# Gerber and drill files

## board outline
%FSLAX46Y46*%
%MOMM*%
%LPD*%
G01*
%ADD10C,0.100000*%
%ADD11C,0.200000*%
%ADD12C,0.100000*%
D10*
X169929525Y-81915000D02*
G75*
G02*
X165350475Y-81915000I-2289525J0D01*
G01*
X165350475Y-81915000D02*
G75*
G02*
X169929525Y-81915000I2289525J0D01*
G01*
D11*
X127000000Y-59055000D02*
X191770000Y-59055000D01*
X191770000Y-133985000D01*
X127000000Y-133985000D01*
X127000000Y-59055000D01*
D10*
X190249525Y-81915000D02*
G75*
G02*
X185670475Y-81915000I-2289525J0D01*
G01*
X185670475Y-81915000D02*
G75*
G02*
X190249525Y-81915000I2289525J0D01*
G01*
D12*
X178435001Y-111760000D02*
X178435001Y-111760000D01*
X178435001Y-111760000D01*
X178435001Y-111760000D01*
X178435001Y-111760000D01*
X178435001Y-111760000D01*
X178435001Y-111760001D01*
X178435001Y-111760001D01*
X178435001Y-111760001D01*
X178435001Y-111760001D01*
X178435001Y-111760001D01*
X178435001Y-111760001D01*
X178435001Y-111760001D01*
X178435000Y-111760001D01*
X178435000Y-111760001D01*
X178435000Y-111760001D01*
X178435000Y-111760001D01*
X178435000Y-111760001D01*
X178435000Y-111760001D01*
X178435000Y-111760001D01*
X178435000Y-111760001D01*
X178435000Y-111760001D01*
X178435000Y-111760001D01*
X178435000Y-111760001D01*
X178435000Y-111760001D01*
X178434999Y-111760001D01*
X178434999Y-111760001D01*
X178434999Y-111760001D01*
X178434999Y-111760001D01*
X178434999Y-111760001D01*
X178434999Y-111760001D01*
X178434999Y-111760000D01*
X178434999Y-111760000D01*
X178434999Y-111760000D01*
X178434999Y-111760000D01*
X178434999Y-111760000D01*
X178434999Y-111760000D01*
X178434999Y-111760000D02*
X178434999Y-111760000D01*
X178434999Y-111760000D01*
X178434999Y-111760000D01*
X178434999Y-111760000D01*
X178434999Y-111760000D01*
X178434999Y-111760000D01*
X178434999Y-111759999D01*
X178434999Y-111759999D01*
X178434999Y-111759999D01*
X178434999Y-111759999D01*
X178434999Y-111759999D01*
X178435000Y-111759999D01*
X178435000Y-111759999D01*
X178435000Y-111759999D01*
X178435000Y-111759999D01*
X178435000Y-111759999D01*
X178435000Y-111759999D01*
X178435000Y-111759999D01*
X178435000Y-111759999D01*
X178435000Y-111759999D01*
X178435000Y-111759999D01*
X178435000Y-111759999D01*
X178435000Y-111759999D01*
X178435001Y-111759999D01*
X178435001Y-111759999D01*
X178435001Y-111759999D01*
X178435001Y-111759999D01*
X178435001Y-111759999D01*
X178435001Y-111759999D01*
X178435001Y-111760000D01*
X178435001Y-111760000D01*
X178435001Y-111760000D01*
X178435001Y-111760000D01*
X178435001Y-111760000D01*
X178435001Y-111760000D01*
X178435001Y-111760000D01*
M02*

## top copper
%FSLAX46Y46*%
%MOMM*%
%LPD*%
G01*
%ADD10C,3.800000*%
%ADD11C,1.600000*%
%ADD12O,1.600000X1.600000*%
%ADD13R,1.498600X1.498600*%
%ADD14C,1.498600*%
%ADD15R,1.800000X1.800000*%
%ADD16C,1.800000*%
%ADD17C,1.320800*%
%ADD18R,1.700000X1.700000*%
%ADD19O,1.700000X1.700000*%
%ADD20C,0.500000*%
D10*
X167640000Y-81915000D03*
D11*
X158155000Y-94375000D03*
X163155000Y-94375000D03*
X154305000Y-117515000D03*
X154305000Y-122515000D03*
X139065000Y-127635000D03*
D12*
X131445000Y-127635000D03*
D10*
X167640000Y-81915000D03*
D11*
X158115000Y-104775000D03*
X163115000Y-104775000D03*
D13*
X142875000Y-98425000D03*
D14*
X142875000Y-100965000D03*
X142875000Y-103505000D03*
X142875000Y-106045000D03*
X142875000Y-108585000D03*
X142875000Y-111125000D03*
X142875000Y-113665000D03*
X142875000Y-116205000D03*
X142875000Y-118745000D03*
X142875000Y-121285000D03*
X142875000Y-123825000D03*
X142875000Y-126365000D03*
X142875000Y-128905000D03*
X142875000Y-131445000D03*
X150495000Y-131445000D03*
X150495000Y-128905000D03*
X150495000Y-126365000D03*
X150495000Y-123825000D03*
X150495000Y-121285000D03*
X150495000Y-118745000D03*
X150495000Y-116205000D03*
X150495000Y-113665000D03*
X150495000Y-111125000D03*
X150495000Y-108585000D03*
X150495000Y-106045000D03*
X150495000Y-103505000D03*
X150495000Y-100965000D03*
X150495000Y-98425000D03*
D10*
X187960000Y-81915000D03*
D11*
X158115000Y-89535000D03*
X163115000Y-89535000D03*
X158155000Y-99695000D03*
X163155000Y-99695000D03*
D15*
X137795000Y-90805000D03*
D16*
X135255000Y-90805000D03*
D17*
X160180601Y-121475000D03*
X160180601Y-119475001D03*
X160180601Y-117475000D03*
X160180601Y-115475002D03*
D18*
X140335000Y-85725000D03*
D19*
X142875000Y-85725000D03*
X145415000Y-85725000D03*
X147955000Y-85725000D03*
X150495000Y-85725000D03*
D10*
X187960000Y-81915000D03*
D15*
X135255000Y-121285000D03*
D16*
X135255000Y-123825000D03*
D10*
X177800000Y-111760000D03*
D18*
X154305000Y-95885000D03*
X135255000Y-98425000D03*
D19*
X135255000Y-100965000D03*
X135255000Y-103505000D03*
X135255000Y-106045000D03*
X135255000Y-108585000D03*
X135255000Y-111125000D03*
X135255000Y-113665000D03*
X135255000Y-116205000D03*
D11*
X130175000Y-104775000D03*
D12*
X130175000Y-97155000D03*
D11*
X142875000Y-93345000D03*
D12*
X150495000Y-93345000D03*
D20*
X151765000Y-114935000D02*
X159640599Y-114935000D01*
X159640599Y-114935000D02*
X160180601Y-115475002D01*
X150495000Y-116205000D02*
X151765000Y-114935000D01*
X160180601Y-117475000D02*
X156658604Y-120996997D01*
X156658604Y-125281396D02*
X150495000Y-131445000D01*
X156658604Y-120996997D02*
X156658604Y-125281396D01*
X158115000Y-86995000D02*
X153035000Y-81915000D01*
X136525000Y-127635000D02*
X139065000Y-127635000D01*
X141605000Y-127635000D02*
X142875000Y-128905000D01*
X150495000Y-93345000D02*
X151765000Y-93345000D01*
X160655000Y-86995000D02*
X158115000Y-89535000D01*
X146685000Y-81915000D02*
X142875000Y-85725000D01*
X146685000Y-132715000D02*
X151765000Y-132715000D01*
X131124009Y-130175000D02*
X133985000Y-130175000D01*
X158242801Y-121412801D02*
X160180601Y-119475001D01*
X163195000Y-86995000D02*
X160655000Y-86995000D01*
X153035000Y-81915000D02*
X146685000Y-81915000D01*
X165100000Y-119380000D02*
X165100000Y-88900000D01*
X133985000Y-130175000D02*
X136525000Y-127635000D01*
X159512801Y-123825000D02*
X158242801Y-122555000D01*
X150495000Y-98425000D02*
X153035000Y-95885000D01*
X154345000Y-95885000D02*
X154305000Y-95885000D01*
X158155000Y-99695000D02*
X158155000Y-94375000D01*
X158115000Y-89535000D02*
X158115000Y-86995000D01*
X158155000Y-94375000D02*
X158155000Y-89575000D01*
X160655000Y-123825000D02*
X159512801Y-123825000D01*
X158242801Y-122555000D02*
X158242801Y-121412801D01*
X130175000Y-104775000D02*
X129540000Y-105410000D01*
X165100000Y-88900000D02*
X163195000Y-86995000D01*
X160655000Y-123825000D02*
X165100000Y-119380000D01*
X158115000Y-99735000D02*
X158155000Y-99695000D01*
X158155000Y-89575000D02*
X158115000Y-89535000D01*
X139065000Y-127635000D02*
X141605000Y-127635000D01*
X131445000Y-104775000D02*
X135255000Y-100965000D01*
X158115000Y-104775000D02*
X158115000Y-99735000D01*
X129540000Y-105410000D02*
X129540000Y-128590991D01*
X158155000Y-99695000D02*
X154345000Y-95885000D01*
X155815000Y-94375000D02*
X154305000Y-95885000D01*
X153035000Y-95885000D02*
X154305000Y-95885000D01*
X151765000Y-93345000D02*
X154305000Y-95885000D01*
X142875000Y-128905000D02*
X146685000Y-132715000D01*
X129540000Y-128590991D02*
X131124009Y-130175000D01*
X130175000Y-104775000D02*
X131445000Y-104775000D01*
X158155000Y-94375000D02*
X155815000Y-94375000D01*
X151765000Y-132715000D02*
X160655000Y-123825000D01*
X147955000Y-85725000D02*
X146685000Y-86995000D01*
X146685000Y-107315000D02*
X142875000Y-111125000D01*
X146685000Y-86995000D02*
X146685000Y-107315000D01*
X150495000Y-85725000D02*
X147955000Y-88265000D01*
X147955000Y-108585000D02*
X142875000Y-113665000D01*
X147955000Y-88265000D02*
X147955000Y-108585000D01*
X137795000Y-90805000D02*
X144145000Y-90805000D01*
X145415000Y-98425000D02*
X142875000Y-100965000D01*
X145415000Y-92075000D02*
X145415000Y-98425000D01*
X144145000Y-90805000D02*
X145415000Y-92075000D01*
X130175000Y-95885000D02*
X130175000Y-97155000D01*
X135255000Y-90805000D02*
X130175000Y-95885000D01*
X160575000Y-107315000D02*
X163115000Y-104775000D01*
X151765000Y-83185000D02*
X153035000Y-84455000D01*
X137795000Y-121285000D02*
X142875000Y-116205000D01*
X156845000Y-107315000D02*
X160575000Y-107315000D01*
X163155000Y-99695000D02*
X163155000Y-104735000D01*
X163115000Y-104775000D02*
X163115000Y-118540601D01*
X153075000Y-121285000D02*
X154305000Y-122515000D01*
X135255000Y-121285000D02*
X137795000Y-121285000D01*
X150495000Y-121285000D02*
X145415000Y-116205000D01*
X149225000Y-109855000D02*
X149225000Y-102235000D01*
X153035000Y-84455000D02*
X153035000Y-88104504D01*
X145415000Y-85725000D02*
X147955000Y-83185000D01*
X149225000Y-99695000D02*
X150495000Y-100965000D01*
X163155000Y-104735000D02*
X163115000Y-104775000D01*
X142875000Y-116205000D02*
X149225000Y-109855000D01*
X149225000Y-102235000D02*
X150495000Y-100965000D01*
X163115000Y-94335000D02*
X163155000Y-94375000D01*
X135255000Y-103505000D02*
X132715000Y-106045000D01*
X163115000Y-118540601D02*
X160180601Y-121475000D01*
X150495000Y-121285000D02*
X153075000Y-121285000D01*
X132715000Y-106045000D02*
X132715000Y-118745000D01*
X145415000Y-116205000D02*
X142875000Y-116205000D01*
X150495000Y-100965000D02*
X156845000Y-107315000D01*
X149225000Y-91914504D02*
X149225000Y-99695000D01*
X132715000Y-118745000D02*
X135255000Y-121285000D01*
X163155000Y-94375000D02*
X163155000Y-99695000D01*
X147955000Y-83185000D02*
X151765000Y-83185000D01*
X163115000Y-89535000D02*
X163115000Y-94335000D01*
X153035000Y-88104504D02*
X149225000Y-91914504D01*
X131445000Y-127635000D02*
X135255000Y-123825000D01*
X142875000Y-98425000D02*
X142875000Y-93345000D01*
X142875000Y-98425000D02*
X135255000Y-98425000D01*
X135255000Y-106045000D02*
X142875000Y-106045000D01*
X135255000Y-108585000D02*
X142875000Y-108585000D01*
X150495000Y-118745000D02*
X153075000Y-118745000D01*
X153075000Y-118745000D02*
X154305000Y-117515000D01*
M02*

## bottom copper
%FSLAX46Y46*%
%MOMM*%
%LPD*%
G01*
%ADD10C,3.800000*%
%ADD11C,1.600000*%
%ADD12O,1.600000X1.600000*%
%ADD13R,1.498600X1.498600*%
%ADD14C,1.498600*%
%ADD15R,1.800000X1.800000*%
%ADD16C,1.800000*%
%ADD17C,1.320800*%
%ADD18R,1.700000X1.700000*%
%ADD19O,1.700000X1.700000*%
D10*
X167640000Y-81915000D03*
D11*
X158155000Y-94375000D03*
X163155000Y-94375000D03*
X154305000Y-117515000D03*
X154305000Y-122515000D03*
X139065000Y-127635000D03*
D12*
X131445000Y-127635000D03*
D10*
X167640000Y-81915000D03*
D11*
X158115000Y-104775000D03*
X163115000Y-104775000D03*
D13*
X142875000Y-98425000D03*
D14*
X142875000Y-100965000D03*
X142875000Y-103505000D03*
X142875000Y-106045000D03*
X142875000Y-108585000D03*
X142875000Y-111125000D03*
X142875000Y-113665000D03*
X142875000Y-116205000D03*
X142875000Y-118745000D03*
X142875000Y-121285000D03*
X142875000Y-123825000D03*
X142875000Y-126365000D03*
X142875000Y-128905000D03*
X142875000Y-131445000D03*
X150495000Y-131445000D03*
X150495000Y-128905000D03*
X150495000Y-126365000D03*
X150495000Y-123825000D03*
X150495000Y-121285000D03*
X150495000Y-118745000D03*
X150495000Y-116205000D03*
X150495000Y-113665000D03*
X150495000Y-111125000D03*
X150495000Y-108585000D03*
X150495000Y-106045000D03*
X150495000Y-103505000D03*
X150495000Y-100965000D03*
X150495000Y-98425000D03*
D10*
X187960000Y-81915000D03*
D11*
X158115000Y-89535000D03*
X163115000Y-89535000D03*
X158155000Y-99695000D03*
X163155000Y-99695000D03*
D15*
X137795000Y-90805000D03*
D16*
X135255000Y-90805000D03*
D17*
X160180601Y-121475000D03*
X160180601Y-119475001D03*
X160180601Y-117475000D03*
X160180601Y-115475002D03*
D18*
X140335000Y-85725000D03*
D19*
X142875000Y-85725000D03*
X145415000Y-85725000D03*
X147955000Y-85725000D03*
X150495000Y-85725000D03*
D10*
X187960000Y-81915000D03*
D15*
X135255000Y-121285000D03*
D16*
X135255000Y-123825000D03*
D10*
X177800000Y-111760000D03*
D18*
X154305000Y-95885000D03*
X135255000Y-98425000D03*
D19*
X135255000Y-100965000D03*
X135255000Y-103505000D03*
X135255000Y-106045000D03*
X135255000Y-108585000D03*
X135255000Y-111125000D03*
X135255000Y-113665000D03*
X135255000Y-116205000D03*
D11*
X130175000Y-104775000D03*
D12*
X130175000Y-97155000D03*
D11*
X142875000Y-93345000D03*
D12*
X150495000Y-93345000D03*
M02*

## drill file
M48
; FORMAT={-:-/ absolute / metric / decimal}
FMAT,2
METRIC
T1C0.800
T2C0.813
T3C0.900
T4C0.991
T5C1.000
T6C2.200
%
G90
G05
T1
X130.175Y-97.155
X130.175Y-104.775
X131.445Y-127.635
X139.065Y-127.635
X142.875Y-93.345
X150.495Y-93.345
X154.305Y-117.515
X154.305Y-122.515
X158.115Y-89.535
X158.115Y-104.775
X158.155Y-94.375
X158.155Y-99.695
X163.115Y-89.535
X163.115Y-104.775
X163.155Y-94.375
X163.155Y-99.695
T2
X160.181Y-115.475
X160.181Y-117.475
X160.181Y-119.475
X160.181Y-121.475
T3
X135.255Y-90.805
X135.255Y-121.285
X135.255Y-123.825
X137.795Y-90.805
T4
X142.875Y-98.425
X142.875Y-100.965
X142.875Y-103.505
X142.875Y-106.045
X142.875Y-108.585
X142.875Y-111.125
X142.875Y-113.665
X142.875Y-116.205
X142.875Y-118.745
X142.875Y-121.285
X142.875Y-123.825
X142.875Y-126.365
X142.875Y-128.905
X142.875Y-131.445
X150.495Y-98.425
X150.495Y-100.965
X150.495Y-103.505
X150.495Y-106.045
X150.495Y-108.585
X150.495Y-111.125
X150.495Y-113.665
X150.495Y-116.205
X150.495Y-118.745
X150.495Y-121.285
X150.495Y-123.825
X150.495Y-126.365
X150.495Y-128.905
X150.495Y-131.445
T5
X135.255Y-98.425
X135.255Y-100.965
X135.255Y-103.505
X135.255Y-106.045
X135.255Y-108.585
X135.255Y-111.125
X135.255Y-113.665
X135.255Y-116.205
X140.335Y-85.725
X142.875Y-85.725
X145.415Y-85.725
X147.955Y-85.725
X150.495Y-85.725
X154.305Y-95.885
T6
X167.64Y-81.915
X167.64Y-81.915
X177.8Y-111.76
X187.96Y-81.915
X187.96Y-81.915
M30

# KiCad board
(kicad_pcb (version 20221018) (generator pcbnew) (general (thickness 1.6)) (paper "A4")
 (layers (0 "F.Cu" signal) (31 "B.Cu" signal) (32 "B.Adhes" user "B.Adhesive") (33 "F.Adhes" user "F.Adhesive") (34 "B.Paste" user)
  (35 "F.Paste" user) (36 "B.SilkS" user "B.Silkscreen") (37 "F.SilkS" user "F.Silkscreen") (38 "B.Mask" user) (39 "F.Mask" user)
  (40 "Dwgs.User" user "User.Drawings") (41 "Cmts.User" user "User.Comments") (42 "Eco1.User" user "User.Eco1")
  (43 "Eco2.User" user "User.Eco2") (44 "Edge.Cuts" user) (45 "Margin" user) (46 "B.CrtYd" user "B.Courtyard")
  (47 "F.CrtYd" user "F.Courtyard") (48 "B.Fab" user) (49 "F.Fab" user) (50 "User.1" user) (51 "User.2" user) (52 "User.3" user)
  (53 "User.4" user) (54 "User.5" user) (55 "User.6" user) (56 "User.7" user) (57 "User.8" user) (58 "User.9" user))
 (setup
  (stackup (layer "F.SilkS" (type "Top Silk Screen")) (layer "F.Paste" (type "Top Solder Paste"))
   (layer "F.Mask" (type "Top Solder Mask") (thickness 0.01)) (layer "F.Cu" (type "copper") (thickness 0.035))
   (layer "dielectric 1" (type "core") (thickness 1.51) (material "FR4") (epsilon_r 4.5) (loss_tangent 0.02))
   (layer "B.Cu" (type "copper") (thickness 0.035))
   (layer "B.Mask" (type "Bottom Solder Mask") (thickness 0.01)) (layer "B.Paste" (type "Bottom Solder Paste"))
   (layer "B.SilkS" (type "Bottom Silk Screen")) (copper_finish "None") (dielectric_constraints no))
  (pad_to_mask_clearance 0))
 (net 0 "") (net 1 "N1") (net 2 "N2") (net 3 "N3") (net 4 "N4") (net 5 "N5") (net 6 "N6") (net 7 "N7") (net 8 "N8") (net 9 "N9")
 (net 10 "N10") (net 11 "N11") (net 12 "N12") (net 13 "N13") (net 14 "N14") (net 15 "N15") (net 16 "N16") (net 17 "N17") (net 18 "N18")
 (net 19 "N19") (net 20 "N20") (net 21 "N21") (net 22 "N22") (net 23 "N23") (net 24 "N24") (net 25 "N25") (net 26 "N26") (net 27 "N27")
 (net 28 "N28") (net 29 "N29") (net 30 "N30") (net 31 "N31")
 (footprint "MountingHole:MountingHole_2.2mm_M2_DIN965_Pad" (layer "F.Cu") (at 167.64 81.915)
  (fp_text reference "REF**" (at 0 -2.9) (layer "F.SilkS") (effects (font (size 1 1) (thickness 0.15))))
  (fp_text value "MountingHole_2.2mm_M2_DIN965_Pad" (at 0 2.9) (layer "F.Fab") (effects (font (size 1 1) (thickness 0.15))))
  (pad "1" thru_hole circle (at 0 0) (size 3.8 3.8) (drill 2.2) (layers "*.Cu" "*.Mask")))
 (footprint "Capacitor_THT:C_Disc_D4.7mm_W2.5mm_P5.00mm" (layer "F.Cu") (at 158.155 94.375)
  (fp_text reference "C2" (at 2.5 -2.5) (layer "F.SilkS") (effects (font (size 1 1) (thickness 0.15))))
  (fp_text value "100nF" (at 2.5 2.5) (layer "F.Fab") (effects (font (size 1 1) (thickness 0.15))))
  (pad "1" thru_hole circle (at 0 0) (size 1.6 1.6) (drill 0.8) (layers "*.Cu" "*.Mask") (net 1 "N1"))
  (pad "2" thru_hole circle (at 5 0) (size 1.6 1.6) (drill 0.8) (layers "*.Cu" "*.Mask") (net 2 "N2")))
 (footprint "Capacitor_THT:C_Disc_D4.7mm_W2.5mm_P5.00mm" (layer "F.Cu") (at 154.305 117.515 -90)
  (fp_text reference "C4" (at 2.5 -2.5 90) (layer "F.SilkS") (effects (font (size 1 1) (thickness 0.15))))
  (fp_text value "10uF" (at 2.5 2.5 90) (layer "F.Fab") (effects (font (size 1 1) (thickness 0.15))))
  (pad "1" thru_hole circle (at 0 0 270) (size 1.6 1.6) (drill 0.8) (layers "*.Cu" "*.Mask") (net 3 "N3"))
  (pad "2" thru_hole circle (at 5 0 270) (size 1.6 1.6) (drill 0.8) (layers "*.Cu" "*.Mask") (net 2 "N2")))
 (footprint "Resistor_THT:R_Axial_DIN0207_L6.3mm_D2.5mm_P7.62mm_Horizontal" (layer "F.Cu") (at 139.065 127.635 180)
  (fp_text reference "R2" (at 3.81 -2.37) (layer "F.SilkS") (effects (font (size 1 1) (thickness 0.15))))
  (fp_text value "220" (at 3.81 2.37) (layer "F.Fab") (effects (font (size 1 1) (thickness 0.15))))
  (pad "1" thru_hole circle (at 0 0 180) (size 1.6 1.6) (drill 0.8) (layers "*.Cu" "*.Mask") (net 1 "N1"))
  (pad "2" thru_hole oval (at 7.62 0 180) (size 1.6 1.6) (drill 0.8) (layers "*.Cu" "*.Mask") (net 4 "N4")))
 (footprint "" (layer "F.Cu") (at 167.64 81.915)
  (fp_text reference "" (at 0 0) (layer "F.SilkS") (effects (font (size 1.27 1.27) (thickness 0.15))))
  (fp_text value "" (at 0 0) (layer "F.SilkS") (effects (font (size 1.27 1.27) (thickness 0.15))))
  (pad "1" thru_hole circle (at 0 0) (size 3.8 3.8) (drill 2.2) (layers "*.Cu" "*.Mask")))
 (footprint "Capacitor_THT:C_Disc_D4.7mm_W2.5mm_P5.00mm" (layer "F.Cu") (at 158.115 104.775)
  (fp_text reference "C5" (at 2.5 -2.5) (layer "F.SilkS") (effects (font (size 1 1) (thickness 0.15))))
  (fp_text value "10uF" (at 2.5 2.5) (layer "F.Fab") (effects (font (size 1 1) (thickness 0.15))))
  (pad "1" thru_hole circle (at 0 0) (size 1.6 1.6) (drill 0.8) (layers "*.Cu" "*.Mask") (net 1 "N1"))
  (pad "2" thru_hole circle (at 5 0) (size 1.6 1.6) (drill 0.8) (layers "*.Cu" "*.Mask") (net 2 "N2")))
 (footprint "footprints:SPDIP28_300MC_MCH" (layer "F.Cu") (at 142.875 98.425)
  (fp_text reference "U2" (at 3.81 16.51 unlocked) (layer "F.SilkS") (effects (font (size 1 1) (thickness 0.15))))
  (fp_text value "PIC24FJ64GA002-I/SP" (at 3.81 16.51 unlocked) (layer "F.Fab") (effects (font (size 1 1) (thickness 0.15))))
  (pad "1" thru_hole rect (at 0 0) (size 1.4986 1.4986) (drill 0.9906) (layers "*.Cu" "*.Mask") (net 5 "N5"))
  (pad "2" thru_hole circle (at 0 2.54) (size 1.4986 1.4986) (drill 0.9906) (layers "*.Cu" "*.Mask") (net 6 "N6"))
  (pad "3" thru_hole circle (at 0 5.08) (size 1.4986 1.4986) (drill 0.9906) (layers "*.Cu" "*.Mask") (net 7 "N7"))
  (pad "4" thru_hole circle (at 0 7.62) (size 1.4986 1.4986) (drill 0.9906) (layers "*.Cu" "*.Mask") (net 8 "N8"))
  (pad "5" thru_hole circle (at 0 10.16) (size 1.4986 1.4986) (drill 0.9906) (layers "*.Cu" "*.Mask") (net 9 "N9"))
  (pad "6" thru_hole circle (at 0 12.7) (size 1.4986 1.4986) (drill 0.9906) (layers "*.Cu" "*.Mask") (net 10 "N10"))
  (pad "7" thru_hole circle (at 0 15.24) (size 1.4986 1.4986) (drill 0.9906) (layers "*.Cu" "*.Mask") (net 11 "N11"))
  (pad "8" thru_hole circle (at 0 17.78) (size 1.4986 1.4986) (drill 0.9906) (layers "*.Cu" "*.Mask") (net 2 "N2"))
  (pad "9" thru_hole circle (at 0 20.32) (size 1.4986 1.4986) (drill 0.9906) (layers "*.Cu" "*.Mask") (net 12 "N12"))
  (pad "10" thru_hole circle (at 0 22.86) (size 1.4986 1.4986) (drill 0.9906) (layers "*.Cu" "*.Mask") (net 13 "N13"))
  (pad "11" thru_hole circle (at 0 25.4) (size 1.4986 1.4986) (drill 0.9906) (layers "*.Cu" "*.Mask") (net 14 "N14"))
  (pad "12" thru_hole circle (at 0 27.94) (size 1.4986 1.4986) (drill 0.9906) (layers "*.Cu" "*.Mask") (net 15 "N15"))
  (pad "13" thru_hole circle (at 0 30.48) (size 1.4986 1.4986) (drill 0.9906) (layers "*.Cu" "*.Mask") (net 1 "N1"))
  (pad "14" thru_hole circle (at 0 33.02) (size 1.4986 1.4986) (drill 0.9906) (layers "*.Cu" "*.Mask") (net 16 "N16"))
  (pad "15" thru_hole circle (at 7.62 33.02) (size 1.4986 1.4986) (drill 0.9906) (layers "*.Cu" "*.Mask") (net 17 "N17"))
  (pad "16" thru_hole circle (at 7.62 30.48) (size 1.4986 1.4986) (drill 0.9906) (layers "*.Cu" "*.Mask") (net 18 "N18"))
  (pad "17" thru_hole circle (at 7.62 27.94) (size 1.4986 1.4986) (drill 0.9906) (layers "*.Cu" "*.Mask") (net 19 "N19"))
  (pad "18" thru_hole circle (at 7.62 25.4) (size 1.4986 1.4986) (drill 0.9906) (layers "*.Cu" "*.Mask") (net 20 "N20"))
  (pad "19" thru_hole circle (at 7.62 22.86) (size 1.4986 1.4986) (drill 0.9906) (layers "*.Cu" "*.Mask") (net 2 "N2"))
  (pad "20" thru_hole circle (at 7.62 20.32) (size 1.4986 1.4986) (drill 0.9906) (layers "*.Cu" "*.Mask") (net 3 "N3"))
  (pad "21" thru_hole circle (at 7.62 17.78) (size 1.4986 1.4986) (drill 0.9906) (layers "*.Cu" "*.Mask") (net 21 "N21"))
  (pad "22" thru_hole circle (at 7.62 15.24) (size 1.4986 1.4986) (drill 0.9906) (layers "*.Cu" "*.Mask") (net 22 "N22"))
  (pad "23" thru_hole circle (at 7.62 12.7) (size 1.4986 1.4986) (drill 0.9906) (layers "*.Cu" "*.Mask") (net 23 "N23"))
  (pad "24" thru_hole circle (at 7.62 10.16) (size 1.4986 1.4986) (drill 0.9906) (layers "*.Cu" "*.Mask") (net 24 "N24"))
  (pad "25" thru_hole circle (at 7.62 7.62) (size 1.4986 1.4986) (drill 0.9906) (layers "*.Cu" "*.Mask") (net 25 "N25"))
  (pad "26" thru_hole circle (at 7.62 5.08) (size 1.4986 1.4986) (drill 0.9906) (layers "*.Cu" "*.Mask") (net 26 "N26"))
  (pad "27" thru_hole circle (at 7.62 2.54) (size 1.4986 1.4986) (drill 0.9906) (layers "*.Cu" "*.Mask") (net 2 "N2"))
  (pad "28" thru_hole circle (at 7.62 0) (size 1.4986 1.4986) (drill 0.9906) (layers "*.Cu" "*.Mask") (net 1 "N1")))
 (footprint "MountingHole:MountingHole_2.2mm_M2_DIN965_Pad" (layer "F.Cu") (at 187.96 81.915)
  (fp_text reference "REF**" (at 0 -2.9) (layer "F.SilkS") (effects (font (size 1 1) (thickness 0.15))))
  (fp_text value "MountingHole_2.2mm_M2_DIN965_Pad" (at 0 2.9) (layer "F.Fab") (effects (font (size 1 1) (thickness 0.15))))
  (pad "1" thru_hole circle (at 0 0) (size 3.8 3.8) (drill 2.2) (layers "*.Cu" "*.Mask")))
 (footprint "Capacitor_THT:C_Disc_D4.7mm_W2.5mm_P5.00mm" (layer "F.Cu") (at 158.115 89.535)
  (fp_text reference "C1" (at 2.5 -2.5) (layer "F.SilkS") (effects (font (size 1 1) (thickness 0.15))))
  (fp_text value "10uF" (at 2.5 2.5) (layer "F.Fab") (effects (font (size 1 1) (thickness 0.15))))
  (pad "1" thru_hole circle (at 0 0) (size 1.6 1.6) (drill 0.8) (layers "*.Cu" "*.Mask") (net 1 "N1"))
  (pad "2" thru_hole circle (at 5 0) (size 1.6 1.6) (drill 0.8) (layers "*.Cu" "*.Mask") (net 2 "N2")))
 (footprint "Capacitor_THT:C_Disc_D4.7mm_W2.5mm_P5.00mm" (layer "F.Cu") (at 158.155 99.695)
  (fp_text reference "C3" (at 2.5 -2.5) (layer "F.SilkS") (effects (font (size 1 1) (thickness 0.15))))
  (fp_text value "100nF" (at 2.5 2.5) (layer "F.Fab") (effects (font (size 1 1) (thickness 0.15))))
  (pad "1" thru_hole circle (at 0 0) (size 1.6 1.6) (drill 0.8) (layers "*.Cu" "*.Mask") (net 1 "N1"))
  (pad "2" thru_hole circle (at 5 0) (size 1.6 1.6) (drill 0.8) (layers "*.Cu" "*.Mask") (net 2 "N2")))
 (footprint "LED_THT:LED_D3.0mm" (layer "F.Cu") (at 137.795 90.805 180)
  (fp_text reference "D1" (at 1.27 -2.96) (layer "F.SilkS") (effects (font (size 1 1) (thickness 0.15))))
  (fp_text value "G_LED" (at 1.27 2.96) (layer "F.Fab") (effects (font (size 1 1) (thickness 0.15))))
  (pad "1" thru_hole rect (at 0 0 180) (size 1.8 1.8) (drill 0.9) (layers "*.Cu" "*.Mask") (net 6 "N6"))
  (pad "2" thru_hole circle (at 2.54 0 180) (size 1.8 1.8) (drill 0.9) (layers "*.Cu" "*.Mask") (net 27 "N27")))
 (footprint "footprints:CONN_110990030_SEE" (layer "F.Cu") (at 160.180601 121.475 90)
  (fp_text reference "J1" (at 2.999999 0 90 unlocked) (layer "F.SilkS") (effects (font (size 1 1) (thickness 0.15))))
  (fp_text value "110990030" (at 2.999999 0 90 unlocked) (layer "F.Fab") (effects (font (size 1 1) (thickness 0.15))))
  (pad "1" thru_hole circle (at 0 0 90) (size 1.3208 1.3208) (drill 0.8128) (layers "*.Cu" "*.Mask") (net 2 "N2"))
  (pad "2" thru_hole circle (at 1.999999 0 90) (size 1.3208 1.3208) (drill 0.8128) (layers "*.Cu" "*.Mask") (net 1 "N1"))
  (pad "3" thru_hole circle (at 4 0 90) (size 1.3208 1.3208) (drill 0.8128) (layers "*.Cu" "*.Mask") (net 17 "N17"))
  (pad "4" thru_hole circle (at 5.999998 0 90) (size 1.3208 1.3208) (drill 0.8128) (layers "*.Cu" "*.Mask") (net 21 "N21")))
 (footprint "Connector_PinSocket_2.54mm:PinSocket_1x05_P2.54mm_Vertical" (layer "F.Cu") (at 140.335 85.725 90)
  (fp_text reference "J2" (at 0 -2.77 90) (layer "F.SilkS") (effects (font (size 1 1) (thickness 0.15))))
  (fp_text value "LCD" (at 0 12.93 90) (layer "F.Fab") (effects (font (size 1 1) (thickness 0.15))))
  (pad "1" thru_hole rect (at 0 0 90) (size 1.7 1.7) (drill 1) (layers "*.Cu" "*.Mask") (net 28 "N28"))
  (pad "2" thru_hole oval (at 0 2.54 90) (size 1.7 1.7) (drill 1) (layers "*.Cu" "*.Mask") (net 1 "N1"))
  (pad "3" thru_hole oval (at 0 5.08 90) (size 1.7 1.7) (drill 1) (layers "*.Cu" "*.Mask") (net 2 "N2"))
  (pad "4" thru_hole oval (at 0 7.62 90) (size 1.7 1.7) (drill 1) (layers "*.Cu" "*.Mask") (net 10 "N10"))
  (pad "5" thru_hole oval (at 0 10.16 90) (size 1.7 1.7) (drill 1) (layers "*.Cu" "*.Mask") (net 11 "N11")))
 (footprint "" (layer "F.Cu") (at 187.96 81.915)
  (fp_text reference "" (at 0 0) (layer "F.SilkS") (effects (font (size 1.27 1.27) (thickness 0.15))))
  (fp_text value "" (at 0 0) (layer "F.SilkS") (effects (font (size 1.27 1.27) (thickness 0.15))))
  (pad "1" thru_hole circle (at 0 0) (size 3.8 3.8) (drill 2.2) (layers "*.Cu" "*.Mask")))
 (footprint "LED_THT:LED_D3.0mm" (layer "F.Cu") (at 135.255 121.285 -90)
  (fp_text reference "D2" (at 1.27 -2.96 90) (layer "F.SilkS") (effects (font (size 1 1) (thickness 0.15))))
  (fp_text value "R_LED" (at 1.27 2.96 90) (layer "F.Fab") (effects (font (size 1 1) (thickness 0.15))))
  (pad "1" thru_hole rect (at 0 0 270) (size 1.8 1.8) (drill 0.9) (layers "*.Cu" "*.Mask") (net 2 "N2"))
  (pad "2" thru_hole circle (at 2.54 0 270) (size 1.8 1.8) (drill 0.9) (layers "*.Cu" "*.Mask") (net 4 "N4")))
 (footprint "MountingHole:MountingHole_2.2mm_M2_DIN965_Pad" (layer "F.Cu") (at 177.8 111.76)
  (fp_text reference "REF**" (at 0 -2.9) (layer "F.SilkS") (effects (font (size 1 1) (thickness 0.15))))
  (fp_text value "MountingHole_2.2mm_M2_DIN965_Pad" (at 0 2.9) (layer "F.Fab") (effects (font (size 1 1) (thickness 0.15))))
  (pad "1" thru_hole circle (at 0 0) (size 3.8 3.8) (drill 2.2) (layers "*.Cu" "*.Mask")))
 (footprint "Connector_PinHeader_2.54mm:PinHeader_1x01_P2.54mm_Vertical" (layer "F.Cu") (at 154.305 95.885)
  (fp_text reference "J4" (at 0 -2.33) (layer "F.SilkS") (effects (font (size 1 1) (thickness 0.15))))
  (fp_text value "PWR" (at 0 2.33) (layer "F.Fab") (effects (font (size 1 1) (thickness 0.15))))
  (pad "1" thru_hole rect (at 0 0) (size 1.7 1.7) (drill 1) (layers "*.Cu" "*.Mask") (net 1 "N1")))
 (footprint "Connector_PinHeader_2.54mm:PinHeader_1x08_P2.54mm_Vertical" (layer "F.Cu") (at 135.255 98.425)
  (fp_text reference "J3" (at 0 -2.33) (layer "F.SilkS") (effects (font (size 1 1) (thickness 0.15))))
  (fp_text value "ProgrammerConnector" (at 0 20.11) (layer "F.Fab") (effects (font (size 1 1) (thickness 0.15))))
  (pad "1" thru_hole rect (at 0 0) (size 1.7 1.7) (drill 1) (layers "*.Cu" "*.Mask") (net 5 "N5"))
  (pad "2" thru_hole oval (at 0 2.54) (size 1.7 1.7) (drill 1) (layers "*.Cu" "*.Mask") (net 1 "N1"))
  (pad "3" thru_hole oval (at 0 5.08) (size 1.7 1.7) (drill 1) (layers "*.Cu" "*.Mask") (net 2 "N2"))
  (pad "4" thru_hole oval (at 0 7.62) (size 1.7 1.7) (drill 1) (layers "*.Cu" "*.Mask") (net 8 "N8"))
  (pad "5" thru_hole oval (at 0 10.16) (size 1.7 1.7) (drill 1) (layers "*.Cu" "*.Mask") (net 9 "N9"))
  (pad "6" thru_hole oval (at 0 12.7) (size 1.7 1.7) (drill 1) (layers "*.Cu" "*.Mask") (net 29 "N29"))
  (pad "7" thru_hole oval (at 0 15.24) (size 1.7 1.7) (drill 1) (layers "*.Cu" "*.Mask") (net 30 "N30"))
  (pad "8" thru_hole oval (at 0 17.78) (size 1.7 1.7) (drill 1) (layers "*.Cu" "*.Mask") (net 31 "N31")))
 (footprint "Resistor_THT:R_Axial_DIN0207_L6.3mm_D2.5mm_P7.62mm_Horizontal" (layer "F.Cu") (at 130.175 104.775 90)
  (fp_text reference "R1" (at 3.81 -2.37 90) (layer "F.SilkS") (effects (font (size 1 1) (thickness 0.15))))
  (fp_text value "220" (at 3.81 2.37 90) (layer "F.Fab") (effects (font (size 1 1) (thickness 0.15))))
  (pad "1" thru_hole circle (at 0 0 90) (size 1.6 1.6) (drill 0.8) (layers "*.Cu" "*.Mask") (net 1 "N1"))
  (pad "2" thru_hole oval (at 7.62 0 90) (size 1.6 1.6) (drill 0.8) (layers "*.Cu" "*.Mask") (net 27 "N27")))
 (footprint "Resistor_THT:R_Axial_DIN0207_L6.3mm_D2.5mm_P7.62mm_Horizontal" (layer "F.Cu") (at 142.875 93.345)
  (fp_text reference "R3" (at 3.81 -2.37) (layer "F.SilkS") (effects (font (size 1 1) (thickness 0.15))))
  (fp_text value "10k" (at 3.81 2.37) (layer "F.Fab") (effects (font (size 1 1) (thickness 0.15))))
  (pad "1" thru_hole circle (at 0 0) (size 1.6 1.6) (drill 0.8) (layers "*.Cu" "*.Mask") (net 5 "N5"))
  (pad "2" thru_hole oval (at 7.62 0) (size 1.6 1.6) (drill 0.8) (layers "*.Cu" "*.Mask") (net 1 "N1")))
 (gr_circle (center 167.64 81.915) (end 169.545 83.185) (stroke (width 0.1) (type default)) (fill none) (layer "Edge.Cuts"))
 (gr_rect (start 127 59.055) (end 191.77 133.985) (stroke (width 0.2) (type default)) (fill none) (layer "Edge.Cuts"))
 (gr_circle (center 187.96 81.915) (end 189.865 83.185) (stroke (width 0.1) (type default)) (fill none) (layer "Edge.Cuts"))
 (gr_circle (center 178.435 111.76) (end 178.435 111.76) (stroke (width 0.1) (type default)) (fill none) (layer "Edge.Cuts"))
 (segment (start 151.765 114.935) (end 159.640599 114.935) (width 0.5) (layer "F.Cu") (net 21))
 (segment (start 159.640599 114.935) (end 160.180601 115.475002) (width 0.5) (layer "F.Cu") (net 21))
 (segment (start 150.495 116.205) (end 151.765 114.935) (width 0.5) (layer "F.Cu") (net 21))
 (segment (start 160.180601 117.475) (end 156.658604 120.996997) (width 0.5) (layer "F.Cu") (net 17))
 (segment (start 156.658604 125.281396) (end 150.495 131.445) (width 0.5) (layer "F.Cu") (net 17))
 (segment (start 156.658604 120.996997) (end 156.658604 125.281396) (width 0.5) (layer "F.Cu") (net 17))
 (segment (start 158.115 86.995) (end 153.035 81.915) (width 0.5) (layer "F.Cu") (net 1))
 (segment (start 136.525 127.635) (end 139.065 127.635) (width 0.5) (layer "F.Cu") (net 1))
 (segment (start 141.605 127.635) (end 142.875 128.905) (width 0.5) (layer "F.Cu") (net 1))
 (segment (start 150.495 93.345) (end 151.765 93.345) (width 0.5) (layer "F.Cu") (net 1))
 (segment (start 160.655 86.995) (end 158.115 89.535) (width 0.5) (layer "F.Cu") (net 1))
 (segment (start 146.685 81.915) (end 142.875 85.725) (width 0.5) (layer "F.Cu") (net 1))
 (segment (start 146.685 132.715) (end 151.765 132.715) (width 0.5) (layer "F.Cu") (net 1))
 (segment (start 131.124009 130.175) (end 133.985 130.175) (width 0.5) (layer "F.Cu") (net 1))
 (segment (start 158.242801 121.412801) (end 160.180601 119.475001) (width 0.5) (layer "F.Cu") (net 1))
 (segment (start 163.195 86.995) (end 160.655 86.995) (width 0.5) (layer "F.Cu") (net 1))
 (segment (start 153.035 81.915) (end 146.685 81.915) (width 0.5) (layer "F.Cu") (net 1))
 (segment (start 165.1 119.38) (end 165.1 88.9) (width 0.5) (layer "F.Cu") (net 1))
 (segment (start 133.985 130.175) (end 136.525 127.635) (width 0.5) (layer "F.Cu") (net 1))
 (segment (start 159.512801 123.825) (end 158.242801 122.555) (width 0.5) (layer "F.Cu") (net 1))
 (segment (start 150.495 98.425) (end 153.035 95.885) (width 0.5) (layer "F.Cu") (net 1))
 (segment (start 154.345 95.885) (end 154.305 95.885) (width 0.5) (layer "F.Cu") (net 1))
 (segment (start 158.155 99.695) (end 158.155 94.375) (width 0.5) (layer "F.Cu") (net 1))
 (segment (start 158.115 89.535) (end 158.115 86.995) (width 0.5) (layer "F.Cu") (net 1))
 (segment (start 158.155 94.375) (end 158.155 89.575) (width 0.5) (layer "F.Cu") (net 1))
 (segment (start 160.655 123.825) (end 159.512801 123.825) (width 0.5) (layer "F.Cu") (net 1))
 (segment (start 158.242801 122.555) (end 158.242801 121.412801) (width 0.5) (layer "F.Cu") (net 1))
 (segment (start 130.175 104.775) (end 129.54 105.41) (width 0.5) (layer "F.Cu") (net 1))
 (segment (start 165.1 88.9) (end 163.195 86.995) (width 0.5) (layer "F.Cu") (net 1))
 (segment (start 160.655 123.825) (end 165.1 119.38) (width 0.5) (layer "F.Cu") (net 1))
 (segment (start 158.115 99.735) (end 158.155 99.695) (width 0.5) (layer "F.Cu") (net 1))
 (segment (start 158.155 89.575) (end 158.115 89.535) (width 0.5) (layer "F.Cu") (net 1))
 (segment (start 139.065 127.635) (end 141.605 127.635) (width 0.5) (layer "F.Cu") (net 1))
 (segment (start 131.445 104.775) (end 135.255 100.965) (width 0.5) (layer "F.Cu") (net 1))
 (segment (start 158.115 104.775) (end 158.115 99.735) (width 0.5) (layer "F.Cu") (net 1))
 (segment (start 129.54 105.41) (end 129.54 128.590991) (width 0.5) (layer "F.Cu") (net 1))
 (segment (start 158.155 99.695) (end 154.345 95.885) (width 0.5) (layer "F.Cu") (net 1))
 (segment (start 155.815 94.375) (end 154.305 95.885) (width 0.5) (layer "F.Cu") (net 1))
 (segment (start 153.035 95.885) (end 154.305 95.885) (width 0.5) (layer "F.Cu") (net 1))
 (segment (start 151.765 93.345) (end 154.305 95.885) (width 0.5) (layer "F.Cu") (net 1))
 (segment (start 142.875 128.905) (end 146.685 132.715) (width 0.5) (layer "F.Cu") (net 1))
 (segment (start 129.54 128.590991) (end 131.124009 130.175) (width 0.5) (layer "F.Cu") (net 1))
 (segment (start 130.175 104.775) (end 131.445 104.775) (width 0.5) (layer "F.Cu") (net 1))
 (segment (start 158.155 94.375) (end 155.815 94.375) (width 0.5) (layer "F.Cu") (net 1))
 (segment (start 151.765 132.715) (end 160.655 123.825) (width 0.5) (layer "F.Cu") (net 1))
 (segment (start 147.955 85.725) (end 146.685 86.995) (width 0.5) (layer "F.Cu") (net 10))
 (segment (start 146.685 107.315) (end 142.875 111.125) (width 0.5) (layer "F.Cu") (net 10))
 (segment (start 146.685 86.995) (end 146.685 107.315) (width 0.5) (layer "F.Cu") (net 10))
 (segment (start 150.495 85.725) (end 147.955 88.265) (width 0.5) (layer "F.Cu") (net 11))
 (segment (start 147.955 108.585) (end 142.875 113.665) (width 0.5) (layer "F.Cu") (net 11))
 (segment (start 147.955 88.265) (end 147.955 108.585) (width 0.5) (layer "F.Cu") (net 11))
 (segment (start 137.795 90.805) (end 144.145 90.805) (width 0.5) (layer "F.Cu") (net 6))
 (segment (start 145.415 98.425) (end 142.875 100.965) (width 0.5) (layer "F.Cu") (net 6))
 (segment (start 145.415 92.075) (end 145.415 98.425) (width 0.5) (layer "F.Cu") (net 6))
 (segment (start 144.145 90.805) (end 145.415 92.075) (width 0.5) (layer "F.Cu") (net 6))
 (segment (start 130.175 95.885) (end 130.175 97.155) (width 0.5) (layer "F.Cu") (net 27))
 (segment (start 135.255 90.805) (end 130.175 95.885) (width 0.5) (layer "F.Cu") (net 27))
 (segment (start 160.575 107.315) (end 163.115 104.775) (width 0.5) (layer "F.Cu") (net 2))
 (segment (start 151.765 83.185) (end 153.035 84.455) (width 0.5) (layer "F.Cu") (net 2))
 (segment (start 137.795 121.285) (end 142.875 116.205) (width 0.5) (layer "F.Cu") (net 2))
 (segment (start 156.845 107.315) (end 160.575 107.315) (width 0.5) (layer "F.Cu") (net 2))
 (segment (start 163.155 99.695) (end 163.155 104.735) (width 0.5) (layer "F.Cu") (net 2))
 (segment (start 163.115 104.775) (end 163.115 118.540601) (width 0.5) (layer "F.Cu") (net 2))
 (segment (start 153.075 121.285) (end 154.305 122.515) (width 0.5) (layer "F.Cu") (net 2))
 (segment (start 135.255 121.285) (end 137.795 121.285) (width 0.5) (layer "F.Cu") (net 2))
 (segment (start 150.495 121.285) (end 145.415 116.205) (width 0.5) (layer "F.Cu") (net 2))
 (segment (start 149.225 109.855) (end 149.225 102.235) (width 0.5) (layer "F.Cu") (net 2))
 (segment (start 153.035 84.455) (end 153.035 88.104504) (width 0.5) (layer "F.Cu") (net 2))
 (segment (start 145.415 85.725) (end 147.955 83.185) (width 0.5) (layer "F.Cu") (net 2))
 (segment (start 149.225 99.695) (end 150.495 100.965) (width 0.5) (layer "F.Cu") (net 2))
 (segment (start 163.155 104.735) (end 163.115 104.775) (width 0.5) (layer "F.Cu") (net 2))
 (segment (start 142.875 116.205) (end 149.225 109.855) (width 0.5) (layer "F.Cu") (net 2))
 (segment (start 149.225 102.235) (end 150.495 100.965) (width 0.5) (layer "F.Cu") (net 2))
 (segment (start 163.115 94.335) (end 163.155 94.375) (width 0.5) (layer "F.Cu") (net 2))
 (segment (start 135.255 103.505) (end 132.715 106.045) (width 0.5) (layer "F.Cu") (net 2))
 (segment (start 163.115 118.540601) (end 160.180601 121.475) (width 0.5) (layer "F.Cu") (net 2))
 (segment (start 150.495 121.285) (end 153.075 121.285) (width 0.5) (layer "F.Cu") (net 2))
 (segment (start 132.715 106.045) (end 132.715 118.745) (width 0.5) (layer "F.Cu") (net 2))
 (segment (start 145.415 116.205) (end 142.875 116.205) (width 0.5) (layer "F.Cu") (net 2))
 (segment (start 150.495 100.965) (end 156.845 107.315) (width 0.5) (layer "F.Cu") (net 2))
 (segment (start 149.225 91.914504) (end 149.225 99.695) (width 0.5) (layer "F.Cu") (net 2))
 (segment (start 132.715 118.745) (end 135.255 121.285) (width 0.5) (layer "F.Cu") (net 2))
 (segment (start 163.155 94.375) (end 163.155 99.695) (width 0.5) (layer "F.Cu") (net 2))
 (segment (start 147.955 83.185) (end 151.765 83.185) (width 0.5) (layer "F.Cu") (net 2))
 (segment (start 163.115 89.535) (end 163.115 94.335) (width 0.5) (layer "F.Cu") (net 2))
 (segment (start 153.035 88.104504) (end 149.225 91.914504) (width 0.5) (layer "F.Cu") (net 2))
 (segment (start 131.445 127.635) (end 135.255 123.825) (width 0.5) (layer "F.Cu") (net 4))
 (segment (start 142.875 98.425) (end 142.875 93.345) (width 0.5) (layer "F.Cu") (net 5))
 (segment (start 142.875 98.425) (end 135.255 98.425) (width 0.5) (layer "F.Cu") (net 5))
 (segment (start 135.255 106.045) (end 142.875 106.045) (width 0.5) (layer "F.Cu") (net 8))
 (segment (start 135.255 108.585) (end 142.875 108.585) (width 0.5) (layer "F.Cu") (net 9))
 (segment (start 150.495 118.745) (end 153.075 118.745) (width 0.5) (layer "F.Cu") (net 3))
 (segment (start 153.075 118.745) (end 154.305 117.515) (width 0.5) (layer "F.Cu") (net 3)))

